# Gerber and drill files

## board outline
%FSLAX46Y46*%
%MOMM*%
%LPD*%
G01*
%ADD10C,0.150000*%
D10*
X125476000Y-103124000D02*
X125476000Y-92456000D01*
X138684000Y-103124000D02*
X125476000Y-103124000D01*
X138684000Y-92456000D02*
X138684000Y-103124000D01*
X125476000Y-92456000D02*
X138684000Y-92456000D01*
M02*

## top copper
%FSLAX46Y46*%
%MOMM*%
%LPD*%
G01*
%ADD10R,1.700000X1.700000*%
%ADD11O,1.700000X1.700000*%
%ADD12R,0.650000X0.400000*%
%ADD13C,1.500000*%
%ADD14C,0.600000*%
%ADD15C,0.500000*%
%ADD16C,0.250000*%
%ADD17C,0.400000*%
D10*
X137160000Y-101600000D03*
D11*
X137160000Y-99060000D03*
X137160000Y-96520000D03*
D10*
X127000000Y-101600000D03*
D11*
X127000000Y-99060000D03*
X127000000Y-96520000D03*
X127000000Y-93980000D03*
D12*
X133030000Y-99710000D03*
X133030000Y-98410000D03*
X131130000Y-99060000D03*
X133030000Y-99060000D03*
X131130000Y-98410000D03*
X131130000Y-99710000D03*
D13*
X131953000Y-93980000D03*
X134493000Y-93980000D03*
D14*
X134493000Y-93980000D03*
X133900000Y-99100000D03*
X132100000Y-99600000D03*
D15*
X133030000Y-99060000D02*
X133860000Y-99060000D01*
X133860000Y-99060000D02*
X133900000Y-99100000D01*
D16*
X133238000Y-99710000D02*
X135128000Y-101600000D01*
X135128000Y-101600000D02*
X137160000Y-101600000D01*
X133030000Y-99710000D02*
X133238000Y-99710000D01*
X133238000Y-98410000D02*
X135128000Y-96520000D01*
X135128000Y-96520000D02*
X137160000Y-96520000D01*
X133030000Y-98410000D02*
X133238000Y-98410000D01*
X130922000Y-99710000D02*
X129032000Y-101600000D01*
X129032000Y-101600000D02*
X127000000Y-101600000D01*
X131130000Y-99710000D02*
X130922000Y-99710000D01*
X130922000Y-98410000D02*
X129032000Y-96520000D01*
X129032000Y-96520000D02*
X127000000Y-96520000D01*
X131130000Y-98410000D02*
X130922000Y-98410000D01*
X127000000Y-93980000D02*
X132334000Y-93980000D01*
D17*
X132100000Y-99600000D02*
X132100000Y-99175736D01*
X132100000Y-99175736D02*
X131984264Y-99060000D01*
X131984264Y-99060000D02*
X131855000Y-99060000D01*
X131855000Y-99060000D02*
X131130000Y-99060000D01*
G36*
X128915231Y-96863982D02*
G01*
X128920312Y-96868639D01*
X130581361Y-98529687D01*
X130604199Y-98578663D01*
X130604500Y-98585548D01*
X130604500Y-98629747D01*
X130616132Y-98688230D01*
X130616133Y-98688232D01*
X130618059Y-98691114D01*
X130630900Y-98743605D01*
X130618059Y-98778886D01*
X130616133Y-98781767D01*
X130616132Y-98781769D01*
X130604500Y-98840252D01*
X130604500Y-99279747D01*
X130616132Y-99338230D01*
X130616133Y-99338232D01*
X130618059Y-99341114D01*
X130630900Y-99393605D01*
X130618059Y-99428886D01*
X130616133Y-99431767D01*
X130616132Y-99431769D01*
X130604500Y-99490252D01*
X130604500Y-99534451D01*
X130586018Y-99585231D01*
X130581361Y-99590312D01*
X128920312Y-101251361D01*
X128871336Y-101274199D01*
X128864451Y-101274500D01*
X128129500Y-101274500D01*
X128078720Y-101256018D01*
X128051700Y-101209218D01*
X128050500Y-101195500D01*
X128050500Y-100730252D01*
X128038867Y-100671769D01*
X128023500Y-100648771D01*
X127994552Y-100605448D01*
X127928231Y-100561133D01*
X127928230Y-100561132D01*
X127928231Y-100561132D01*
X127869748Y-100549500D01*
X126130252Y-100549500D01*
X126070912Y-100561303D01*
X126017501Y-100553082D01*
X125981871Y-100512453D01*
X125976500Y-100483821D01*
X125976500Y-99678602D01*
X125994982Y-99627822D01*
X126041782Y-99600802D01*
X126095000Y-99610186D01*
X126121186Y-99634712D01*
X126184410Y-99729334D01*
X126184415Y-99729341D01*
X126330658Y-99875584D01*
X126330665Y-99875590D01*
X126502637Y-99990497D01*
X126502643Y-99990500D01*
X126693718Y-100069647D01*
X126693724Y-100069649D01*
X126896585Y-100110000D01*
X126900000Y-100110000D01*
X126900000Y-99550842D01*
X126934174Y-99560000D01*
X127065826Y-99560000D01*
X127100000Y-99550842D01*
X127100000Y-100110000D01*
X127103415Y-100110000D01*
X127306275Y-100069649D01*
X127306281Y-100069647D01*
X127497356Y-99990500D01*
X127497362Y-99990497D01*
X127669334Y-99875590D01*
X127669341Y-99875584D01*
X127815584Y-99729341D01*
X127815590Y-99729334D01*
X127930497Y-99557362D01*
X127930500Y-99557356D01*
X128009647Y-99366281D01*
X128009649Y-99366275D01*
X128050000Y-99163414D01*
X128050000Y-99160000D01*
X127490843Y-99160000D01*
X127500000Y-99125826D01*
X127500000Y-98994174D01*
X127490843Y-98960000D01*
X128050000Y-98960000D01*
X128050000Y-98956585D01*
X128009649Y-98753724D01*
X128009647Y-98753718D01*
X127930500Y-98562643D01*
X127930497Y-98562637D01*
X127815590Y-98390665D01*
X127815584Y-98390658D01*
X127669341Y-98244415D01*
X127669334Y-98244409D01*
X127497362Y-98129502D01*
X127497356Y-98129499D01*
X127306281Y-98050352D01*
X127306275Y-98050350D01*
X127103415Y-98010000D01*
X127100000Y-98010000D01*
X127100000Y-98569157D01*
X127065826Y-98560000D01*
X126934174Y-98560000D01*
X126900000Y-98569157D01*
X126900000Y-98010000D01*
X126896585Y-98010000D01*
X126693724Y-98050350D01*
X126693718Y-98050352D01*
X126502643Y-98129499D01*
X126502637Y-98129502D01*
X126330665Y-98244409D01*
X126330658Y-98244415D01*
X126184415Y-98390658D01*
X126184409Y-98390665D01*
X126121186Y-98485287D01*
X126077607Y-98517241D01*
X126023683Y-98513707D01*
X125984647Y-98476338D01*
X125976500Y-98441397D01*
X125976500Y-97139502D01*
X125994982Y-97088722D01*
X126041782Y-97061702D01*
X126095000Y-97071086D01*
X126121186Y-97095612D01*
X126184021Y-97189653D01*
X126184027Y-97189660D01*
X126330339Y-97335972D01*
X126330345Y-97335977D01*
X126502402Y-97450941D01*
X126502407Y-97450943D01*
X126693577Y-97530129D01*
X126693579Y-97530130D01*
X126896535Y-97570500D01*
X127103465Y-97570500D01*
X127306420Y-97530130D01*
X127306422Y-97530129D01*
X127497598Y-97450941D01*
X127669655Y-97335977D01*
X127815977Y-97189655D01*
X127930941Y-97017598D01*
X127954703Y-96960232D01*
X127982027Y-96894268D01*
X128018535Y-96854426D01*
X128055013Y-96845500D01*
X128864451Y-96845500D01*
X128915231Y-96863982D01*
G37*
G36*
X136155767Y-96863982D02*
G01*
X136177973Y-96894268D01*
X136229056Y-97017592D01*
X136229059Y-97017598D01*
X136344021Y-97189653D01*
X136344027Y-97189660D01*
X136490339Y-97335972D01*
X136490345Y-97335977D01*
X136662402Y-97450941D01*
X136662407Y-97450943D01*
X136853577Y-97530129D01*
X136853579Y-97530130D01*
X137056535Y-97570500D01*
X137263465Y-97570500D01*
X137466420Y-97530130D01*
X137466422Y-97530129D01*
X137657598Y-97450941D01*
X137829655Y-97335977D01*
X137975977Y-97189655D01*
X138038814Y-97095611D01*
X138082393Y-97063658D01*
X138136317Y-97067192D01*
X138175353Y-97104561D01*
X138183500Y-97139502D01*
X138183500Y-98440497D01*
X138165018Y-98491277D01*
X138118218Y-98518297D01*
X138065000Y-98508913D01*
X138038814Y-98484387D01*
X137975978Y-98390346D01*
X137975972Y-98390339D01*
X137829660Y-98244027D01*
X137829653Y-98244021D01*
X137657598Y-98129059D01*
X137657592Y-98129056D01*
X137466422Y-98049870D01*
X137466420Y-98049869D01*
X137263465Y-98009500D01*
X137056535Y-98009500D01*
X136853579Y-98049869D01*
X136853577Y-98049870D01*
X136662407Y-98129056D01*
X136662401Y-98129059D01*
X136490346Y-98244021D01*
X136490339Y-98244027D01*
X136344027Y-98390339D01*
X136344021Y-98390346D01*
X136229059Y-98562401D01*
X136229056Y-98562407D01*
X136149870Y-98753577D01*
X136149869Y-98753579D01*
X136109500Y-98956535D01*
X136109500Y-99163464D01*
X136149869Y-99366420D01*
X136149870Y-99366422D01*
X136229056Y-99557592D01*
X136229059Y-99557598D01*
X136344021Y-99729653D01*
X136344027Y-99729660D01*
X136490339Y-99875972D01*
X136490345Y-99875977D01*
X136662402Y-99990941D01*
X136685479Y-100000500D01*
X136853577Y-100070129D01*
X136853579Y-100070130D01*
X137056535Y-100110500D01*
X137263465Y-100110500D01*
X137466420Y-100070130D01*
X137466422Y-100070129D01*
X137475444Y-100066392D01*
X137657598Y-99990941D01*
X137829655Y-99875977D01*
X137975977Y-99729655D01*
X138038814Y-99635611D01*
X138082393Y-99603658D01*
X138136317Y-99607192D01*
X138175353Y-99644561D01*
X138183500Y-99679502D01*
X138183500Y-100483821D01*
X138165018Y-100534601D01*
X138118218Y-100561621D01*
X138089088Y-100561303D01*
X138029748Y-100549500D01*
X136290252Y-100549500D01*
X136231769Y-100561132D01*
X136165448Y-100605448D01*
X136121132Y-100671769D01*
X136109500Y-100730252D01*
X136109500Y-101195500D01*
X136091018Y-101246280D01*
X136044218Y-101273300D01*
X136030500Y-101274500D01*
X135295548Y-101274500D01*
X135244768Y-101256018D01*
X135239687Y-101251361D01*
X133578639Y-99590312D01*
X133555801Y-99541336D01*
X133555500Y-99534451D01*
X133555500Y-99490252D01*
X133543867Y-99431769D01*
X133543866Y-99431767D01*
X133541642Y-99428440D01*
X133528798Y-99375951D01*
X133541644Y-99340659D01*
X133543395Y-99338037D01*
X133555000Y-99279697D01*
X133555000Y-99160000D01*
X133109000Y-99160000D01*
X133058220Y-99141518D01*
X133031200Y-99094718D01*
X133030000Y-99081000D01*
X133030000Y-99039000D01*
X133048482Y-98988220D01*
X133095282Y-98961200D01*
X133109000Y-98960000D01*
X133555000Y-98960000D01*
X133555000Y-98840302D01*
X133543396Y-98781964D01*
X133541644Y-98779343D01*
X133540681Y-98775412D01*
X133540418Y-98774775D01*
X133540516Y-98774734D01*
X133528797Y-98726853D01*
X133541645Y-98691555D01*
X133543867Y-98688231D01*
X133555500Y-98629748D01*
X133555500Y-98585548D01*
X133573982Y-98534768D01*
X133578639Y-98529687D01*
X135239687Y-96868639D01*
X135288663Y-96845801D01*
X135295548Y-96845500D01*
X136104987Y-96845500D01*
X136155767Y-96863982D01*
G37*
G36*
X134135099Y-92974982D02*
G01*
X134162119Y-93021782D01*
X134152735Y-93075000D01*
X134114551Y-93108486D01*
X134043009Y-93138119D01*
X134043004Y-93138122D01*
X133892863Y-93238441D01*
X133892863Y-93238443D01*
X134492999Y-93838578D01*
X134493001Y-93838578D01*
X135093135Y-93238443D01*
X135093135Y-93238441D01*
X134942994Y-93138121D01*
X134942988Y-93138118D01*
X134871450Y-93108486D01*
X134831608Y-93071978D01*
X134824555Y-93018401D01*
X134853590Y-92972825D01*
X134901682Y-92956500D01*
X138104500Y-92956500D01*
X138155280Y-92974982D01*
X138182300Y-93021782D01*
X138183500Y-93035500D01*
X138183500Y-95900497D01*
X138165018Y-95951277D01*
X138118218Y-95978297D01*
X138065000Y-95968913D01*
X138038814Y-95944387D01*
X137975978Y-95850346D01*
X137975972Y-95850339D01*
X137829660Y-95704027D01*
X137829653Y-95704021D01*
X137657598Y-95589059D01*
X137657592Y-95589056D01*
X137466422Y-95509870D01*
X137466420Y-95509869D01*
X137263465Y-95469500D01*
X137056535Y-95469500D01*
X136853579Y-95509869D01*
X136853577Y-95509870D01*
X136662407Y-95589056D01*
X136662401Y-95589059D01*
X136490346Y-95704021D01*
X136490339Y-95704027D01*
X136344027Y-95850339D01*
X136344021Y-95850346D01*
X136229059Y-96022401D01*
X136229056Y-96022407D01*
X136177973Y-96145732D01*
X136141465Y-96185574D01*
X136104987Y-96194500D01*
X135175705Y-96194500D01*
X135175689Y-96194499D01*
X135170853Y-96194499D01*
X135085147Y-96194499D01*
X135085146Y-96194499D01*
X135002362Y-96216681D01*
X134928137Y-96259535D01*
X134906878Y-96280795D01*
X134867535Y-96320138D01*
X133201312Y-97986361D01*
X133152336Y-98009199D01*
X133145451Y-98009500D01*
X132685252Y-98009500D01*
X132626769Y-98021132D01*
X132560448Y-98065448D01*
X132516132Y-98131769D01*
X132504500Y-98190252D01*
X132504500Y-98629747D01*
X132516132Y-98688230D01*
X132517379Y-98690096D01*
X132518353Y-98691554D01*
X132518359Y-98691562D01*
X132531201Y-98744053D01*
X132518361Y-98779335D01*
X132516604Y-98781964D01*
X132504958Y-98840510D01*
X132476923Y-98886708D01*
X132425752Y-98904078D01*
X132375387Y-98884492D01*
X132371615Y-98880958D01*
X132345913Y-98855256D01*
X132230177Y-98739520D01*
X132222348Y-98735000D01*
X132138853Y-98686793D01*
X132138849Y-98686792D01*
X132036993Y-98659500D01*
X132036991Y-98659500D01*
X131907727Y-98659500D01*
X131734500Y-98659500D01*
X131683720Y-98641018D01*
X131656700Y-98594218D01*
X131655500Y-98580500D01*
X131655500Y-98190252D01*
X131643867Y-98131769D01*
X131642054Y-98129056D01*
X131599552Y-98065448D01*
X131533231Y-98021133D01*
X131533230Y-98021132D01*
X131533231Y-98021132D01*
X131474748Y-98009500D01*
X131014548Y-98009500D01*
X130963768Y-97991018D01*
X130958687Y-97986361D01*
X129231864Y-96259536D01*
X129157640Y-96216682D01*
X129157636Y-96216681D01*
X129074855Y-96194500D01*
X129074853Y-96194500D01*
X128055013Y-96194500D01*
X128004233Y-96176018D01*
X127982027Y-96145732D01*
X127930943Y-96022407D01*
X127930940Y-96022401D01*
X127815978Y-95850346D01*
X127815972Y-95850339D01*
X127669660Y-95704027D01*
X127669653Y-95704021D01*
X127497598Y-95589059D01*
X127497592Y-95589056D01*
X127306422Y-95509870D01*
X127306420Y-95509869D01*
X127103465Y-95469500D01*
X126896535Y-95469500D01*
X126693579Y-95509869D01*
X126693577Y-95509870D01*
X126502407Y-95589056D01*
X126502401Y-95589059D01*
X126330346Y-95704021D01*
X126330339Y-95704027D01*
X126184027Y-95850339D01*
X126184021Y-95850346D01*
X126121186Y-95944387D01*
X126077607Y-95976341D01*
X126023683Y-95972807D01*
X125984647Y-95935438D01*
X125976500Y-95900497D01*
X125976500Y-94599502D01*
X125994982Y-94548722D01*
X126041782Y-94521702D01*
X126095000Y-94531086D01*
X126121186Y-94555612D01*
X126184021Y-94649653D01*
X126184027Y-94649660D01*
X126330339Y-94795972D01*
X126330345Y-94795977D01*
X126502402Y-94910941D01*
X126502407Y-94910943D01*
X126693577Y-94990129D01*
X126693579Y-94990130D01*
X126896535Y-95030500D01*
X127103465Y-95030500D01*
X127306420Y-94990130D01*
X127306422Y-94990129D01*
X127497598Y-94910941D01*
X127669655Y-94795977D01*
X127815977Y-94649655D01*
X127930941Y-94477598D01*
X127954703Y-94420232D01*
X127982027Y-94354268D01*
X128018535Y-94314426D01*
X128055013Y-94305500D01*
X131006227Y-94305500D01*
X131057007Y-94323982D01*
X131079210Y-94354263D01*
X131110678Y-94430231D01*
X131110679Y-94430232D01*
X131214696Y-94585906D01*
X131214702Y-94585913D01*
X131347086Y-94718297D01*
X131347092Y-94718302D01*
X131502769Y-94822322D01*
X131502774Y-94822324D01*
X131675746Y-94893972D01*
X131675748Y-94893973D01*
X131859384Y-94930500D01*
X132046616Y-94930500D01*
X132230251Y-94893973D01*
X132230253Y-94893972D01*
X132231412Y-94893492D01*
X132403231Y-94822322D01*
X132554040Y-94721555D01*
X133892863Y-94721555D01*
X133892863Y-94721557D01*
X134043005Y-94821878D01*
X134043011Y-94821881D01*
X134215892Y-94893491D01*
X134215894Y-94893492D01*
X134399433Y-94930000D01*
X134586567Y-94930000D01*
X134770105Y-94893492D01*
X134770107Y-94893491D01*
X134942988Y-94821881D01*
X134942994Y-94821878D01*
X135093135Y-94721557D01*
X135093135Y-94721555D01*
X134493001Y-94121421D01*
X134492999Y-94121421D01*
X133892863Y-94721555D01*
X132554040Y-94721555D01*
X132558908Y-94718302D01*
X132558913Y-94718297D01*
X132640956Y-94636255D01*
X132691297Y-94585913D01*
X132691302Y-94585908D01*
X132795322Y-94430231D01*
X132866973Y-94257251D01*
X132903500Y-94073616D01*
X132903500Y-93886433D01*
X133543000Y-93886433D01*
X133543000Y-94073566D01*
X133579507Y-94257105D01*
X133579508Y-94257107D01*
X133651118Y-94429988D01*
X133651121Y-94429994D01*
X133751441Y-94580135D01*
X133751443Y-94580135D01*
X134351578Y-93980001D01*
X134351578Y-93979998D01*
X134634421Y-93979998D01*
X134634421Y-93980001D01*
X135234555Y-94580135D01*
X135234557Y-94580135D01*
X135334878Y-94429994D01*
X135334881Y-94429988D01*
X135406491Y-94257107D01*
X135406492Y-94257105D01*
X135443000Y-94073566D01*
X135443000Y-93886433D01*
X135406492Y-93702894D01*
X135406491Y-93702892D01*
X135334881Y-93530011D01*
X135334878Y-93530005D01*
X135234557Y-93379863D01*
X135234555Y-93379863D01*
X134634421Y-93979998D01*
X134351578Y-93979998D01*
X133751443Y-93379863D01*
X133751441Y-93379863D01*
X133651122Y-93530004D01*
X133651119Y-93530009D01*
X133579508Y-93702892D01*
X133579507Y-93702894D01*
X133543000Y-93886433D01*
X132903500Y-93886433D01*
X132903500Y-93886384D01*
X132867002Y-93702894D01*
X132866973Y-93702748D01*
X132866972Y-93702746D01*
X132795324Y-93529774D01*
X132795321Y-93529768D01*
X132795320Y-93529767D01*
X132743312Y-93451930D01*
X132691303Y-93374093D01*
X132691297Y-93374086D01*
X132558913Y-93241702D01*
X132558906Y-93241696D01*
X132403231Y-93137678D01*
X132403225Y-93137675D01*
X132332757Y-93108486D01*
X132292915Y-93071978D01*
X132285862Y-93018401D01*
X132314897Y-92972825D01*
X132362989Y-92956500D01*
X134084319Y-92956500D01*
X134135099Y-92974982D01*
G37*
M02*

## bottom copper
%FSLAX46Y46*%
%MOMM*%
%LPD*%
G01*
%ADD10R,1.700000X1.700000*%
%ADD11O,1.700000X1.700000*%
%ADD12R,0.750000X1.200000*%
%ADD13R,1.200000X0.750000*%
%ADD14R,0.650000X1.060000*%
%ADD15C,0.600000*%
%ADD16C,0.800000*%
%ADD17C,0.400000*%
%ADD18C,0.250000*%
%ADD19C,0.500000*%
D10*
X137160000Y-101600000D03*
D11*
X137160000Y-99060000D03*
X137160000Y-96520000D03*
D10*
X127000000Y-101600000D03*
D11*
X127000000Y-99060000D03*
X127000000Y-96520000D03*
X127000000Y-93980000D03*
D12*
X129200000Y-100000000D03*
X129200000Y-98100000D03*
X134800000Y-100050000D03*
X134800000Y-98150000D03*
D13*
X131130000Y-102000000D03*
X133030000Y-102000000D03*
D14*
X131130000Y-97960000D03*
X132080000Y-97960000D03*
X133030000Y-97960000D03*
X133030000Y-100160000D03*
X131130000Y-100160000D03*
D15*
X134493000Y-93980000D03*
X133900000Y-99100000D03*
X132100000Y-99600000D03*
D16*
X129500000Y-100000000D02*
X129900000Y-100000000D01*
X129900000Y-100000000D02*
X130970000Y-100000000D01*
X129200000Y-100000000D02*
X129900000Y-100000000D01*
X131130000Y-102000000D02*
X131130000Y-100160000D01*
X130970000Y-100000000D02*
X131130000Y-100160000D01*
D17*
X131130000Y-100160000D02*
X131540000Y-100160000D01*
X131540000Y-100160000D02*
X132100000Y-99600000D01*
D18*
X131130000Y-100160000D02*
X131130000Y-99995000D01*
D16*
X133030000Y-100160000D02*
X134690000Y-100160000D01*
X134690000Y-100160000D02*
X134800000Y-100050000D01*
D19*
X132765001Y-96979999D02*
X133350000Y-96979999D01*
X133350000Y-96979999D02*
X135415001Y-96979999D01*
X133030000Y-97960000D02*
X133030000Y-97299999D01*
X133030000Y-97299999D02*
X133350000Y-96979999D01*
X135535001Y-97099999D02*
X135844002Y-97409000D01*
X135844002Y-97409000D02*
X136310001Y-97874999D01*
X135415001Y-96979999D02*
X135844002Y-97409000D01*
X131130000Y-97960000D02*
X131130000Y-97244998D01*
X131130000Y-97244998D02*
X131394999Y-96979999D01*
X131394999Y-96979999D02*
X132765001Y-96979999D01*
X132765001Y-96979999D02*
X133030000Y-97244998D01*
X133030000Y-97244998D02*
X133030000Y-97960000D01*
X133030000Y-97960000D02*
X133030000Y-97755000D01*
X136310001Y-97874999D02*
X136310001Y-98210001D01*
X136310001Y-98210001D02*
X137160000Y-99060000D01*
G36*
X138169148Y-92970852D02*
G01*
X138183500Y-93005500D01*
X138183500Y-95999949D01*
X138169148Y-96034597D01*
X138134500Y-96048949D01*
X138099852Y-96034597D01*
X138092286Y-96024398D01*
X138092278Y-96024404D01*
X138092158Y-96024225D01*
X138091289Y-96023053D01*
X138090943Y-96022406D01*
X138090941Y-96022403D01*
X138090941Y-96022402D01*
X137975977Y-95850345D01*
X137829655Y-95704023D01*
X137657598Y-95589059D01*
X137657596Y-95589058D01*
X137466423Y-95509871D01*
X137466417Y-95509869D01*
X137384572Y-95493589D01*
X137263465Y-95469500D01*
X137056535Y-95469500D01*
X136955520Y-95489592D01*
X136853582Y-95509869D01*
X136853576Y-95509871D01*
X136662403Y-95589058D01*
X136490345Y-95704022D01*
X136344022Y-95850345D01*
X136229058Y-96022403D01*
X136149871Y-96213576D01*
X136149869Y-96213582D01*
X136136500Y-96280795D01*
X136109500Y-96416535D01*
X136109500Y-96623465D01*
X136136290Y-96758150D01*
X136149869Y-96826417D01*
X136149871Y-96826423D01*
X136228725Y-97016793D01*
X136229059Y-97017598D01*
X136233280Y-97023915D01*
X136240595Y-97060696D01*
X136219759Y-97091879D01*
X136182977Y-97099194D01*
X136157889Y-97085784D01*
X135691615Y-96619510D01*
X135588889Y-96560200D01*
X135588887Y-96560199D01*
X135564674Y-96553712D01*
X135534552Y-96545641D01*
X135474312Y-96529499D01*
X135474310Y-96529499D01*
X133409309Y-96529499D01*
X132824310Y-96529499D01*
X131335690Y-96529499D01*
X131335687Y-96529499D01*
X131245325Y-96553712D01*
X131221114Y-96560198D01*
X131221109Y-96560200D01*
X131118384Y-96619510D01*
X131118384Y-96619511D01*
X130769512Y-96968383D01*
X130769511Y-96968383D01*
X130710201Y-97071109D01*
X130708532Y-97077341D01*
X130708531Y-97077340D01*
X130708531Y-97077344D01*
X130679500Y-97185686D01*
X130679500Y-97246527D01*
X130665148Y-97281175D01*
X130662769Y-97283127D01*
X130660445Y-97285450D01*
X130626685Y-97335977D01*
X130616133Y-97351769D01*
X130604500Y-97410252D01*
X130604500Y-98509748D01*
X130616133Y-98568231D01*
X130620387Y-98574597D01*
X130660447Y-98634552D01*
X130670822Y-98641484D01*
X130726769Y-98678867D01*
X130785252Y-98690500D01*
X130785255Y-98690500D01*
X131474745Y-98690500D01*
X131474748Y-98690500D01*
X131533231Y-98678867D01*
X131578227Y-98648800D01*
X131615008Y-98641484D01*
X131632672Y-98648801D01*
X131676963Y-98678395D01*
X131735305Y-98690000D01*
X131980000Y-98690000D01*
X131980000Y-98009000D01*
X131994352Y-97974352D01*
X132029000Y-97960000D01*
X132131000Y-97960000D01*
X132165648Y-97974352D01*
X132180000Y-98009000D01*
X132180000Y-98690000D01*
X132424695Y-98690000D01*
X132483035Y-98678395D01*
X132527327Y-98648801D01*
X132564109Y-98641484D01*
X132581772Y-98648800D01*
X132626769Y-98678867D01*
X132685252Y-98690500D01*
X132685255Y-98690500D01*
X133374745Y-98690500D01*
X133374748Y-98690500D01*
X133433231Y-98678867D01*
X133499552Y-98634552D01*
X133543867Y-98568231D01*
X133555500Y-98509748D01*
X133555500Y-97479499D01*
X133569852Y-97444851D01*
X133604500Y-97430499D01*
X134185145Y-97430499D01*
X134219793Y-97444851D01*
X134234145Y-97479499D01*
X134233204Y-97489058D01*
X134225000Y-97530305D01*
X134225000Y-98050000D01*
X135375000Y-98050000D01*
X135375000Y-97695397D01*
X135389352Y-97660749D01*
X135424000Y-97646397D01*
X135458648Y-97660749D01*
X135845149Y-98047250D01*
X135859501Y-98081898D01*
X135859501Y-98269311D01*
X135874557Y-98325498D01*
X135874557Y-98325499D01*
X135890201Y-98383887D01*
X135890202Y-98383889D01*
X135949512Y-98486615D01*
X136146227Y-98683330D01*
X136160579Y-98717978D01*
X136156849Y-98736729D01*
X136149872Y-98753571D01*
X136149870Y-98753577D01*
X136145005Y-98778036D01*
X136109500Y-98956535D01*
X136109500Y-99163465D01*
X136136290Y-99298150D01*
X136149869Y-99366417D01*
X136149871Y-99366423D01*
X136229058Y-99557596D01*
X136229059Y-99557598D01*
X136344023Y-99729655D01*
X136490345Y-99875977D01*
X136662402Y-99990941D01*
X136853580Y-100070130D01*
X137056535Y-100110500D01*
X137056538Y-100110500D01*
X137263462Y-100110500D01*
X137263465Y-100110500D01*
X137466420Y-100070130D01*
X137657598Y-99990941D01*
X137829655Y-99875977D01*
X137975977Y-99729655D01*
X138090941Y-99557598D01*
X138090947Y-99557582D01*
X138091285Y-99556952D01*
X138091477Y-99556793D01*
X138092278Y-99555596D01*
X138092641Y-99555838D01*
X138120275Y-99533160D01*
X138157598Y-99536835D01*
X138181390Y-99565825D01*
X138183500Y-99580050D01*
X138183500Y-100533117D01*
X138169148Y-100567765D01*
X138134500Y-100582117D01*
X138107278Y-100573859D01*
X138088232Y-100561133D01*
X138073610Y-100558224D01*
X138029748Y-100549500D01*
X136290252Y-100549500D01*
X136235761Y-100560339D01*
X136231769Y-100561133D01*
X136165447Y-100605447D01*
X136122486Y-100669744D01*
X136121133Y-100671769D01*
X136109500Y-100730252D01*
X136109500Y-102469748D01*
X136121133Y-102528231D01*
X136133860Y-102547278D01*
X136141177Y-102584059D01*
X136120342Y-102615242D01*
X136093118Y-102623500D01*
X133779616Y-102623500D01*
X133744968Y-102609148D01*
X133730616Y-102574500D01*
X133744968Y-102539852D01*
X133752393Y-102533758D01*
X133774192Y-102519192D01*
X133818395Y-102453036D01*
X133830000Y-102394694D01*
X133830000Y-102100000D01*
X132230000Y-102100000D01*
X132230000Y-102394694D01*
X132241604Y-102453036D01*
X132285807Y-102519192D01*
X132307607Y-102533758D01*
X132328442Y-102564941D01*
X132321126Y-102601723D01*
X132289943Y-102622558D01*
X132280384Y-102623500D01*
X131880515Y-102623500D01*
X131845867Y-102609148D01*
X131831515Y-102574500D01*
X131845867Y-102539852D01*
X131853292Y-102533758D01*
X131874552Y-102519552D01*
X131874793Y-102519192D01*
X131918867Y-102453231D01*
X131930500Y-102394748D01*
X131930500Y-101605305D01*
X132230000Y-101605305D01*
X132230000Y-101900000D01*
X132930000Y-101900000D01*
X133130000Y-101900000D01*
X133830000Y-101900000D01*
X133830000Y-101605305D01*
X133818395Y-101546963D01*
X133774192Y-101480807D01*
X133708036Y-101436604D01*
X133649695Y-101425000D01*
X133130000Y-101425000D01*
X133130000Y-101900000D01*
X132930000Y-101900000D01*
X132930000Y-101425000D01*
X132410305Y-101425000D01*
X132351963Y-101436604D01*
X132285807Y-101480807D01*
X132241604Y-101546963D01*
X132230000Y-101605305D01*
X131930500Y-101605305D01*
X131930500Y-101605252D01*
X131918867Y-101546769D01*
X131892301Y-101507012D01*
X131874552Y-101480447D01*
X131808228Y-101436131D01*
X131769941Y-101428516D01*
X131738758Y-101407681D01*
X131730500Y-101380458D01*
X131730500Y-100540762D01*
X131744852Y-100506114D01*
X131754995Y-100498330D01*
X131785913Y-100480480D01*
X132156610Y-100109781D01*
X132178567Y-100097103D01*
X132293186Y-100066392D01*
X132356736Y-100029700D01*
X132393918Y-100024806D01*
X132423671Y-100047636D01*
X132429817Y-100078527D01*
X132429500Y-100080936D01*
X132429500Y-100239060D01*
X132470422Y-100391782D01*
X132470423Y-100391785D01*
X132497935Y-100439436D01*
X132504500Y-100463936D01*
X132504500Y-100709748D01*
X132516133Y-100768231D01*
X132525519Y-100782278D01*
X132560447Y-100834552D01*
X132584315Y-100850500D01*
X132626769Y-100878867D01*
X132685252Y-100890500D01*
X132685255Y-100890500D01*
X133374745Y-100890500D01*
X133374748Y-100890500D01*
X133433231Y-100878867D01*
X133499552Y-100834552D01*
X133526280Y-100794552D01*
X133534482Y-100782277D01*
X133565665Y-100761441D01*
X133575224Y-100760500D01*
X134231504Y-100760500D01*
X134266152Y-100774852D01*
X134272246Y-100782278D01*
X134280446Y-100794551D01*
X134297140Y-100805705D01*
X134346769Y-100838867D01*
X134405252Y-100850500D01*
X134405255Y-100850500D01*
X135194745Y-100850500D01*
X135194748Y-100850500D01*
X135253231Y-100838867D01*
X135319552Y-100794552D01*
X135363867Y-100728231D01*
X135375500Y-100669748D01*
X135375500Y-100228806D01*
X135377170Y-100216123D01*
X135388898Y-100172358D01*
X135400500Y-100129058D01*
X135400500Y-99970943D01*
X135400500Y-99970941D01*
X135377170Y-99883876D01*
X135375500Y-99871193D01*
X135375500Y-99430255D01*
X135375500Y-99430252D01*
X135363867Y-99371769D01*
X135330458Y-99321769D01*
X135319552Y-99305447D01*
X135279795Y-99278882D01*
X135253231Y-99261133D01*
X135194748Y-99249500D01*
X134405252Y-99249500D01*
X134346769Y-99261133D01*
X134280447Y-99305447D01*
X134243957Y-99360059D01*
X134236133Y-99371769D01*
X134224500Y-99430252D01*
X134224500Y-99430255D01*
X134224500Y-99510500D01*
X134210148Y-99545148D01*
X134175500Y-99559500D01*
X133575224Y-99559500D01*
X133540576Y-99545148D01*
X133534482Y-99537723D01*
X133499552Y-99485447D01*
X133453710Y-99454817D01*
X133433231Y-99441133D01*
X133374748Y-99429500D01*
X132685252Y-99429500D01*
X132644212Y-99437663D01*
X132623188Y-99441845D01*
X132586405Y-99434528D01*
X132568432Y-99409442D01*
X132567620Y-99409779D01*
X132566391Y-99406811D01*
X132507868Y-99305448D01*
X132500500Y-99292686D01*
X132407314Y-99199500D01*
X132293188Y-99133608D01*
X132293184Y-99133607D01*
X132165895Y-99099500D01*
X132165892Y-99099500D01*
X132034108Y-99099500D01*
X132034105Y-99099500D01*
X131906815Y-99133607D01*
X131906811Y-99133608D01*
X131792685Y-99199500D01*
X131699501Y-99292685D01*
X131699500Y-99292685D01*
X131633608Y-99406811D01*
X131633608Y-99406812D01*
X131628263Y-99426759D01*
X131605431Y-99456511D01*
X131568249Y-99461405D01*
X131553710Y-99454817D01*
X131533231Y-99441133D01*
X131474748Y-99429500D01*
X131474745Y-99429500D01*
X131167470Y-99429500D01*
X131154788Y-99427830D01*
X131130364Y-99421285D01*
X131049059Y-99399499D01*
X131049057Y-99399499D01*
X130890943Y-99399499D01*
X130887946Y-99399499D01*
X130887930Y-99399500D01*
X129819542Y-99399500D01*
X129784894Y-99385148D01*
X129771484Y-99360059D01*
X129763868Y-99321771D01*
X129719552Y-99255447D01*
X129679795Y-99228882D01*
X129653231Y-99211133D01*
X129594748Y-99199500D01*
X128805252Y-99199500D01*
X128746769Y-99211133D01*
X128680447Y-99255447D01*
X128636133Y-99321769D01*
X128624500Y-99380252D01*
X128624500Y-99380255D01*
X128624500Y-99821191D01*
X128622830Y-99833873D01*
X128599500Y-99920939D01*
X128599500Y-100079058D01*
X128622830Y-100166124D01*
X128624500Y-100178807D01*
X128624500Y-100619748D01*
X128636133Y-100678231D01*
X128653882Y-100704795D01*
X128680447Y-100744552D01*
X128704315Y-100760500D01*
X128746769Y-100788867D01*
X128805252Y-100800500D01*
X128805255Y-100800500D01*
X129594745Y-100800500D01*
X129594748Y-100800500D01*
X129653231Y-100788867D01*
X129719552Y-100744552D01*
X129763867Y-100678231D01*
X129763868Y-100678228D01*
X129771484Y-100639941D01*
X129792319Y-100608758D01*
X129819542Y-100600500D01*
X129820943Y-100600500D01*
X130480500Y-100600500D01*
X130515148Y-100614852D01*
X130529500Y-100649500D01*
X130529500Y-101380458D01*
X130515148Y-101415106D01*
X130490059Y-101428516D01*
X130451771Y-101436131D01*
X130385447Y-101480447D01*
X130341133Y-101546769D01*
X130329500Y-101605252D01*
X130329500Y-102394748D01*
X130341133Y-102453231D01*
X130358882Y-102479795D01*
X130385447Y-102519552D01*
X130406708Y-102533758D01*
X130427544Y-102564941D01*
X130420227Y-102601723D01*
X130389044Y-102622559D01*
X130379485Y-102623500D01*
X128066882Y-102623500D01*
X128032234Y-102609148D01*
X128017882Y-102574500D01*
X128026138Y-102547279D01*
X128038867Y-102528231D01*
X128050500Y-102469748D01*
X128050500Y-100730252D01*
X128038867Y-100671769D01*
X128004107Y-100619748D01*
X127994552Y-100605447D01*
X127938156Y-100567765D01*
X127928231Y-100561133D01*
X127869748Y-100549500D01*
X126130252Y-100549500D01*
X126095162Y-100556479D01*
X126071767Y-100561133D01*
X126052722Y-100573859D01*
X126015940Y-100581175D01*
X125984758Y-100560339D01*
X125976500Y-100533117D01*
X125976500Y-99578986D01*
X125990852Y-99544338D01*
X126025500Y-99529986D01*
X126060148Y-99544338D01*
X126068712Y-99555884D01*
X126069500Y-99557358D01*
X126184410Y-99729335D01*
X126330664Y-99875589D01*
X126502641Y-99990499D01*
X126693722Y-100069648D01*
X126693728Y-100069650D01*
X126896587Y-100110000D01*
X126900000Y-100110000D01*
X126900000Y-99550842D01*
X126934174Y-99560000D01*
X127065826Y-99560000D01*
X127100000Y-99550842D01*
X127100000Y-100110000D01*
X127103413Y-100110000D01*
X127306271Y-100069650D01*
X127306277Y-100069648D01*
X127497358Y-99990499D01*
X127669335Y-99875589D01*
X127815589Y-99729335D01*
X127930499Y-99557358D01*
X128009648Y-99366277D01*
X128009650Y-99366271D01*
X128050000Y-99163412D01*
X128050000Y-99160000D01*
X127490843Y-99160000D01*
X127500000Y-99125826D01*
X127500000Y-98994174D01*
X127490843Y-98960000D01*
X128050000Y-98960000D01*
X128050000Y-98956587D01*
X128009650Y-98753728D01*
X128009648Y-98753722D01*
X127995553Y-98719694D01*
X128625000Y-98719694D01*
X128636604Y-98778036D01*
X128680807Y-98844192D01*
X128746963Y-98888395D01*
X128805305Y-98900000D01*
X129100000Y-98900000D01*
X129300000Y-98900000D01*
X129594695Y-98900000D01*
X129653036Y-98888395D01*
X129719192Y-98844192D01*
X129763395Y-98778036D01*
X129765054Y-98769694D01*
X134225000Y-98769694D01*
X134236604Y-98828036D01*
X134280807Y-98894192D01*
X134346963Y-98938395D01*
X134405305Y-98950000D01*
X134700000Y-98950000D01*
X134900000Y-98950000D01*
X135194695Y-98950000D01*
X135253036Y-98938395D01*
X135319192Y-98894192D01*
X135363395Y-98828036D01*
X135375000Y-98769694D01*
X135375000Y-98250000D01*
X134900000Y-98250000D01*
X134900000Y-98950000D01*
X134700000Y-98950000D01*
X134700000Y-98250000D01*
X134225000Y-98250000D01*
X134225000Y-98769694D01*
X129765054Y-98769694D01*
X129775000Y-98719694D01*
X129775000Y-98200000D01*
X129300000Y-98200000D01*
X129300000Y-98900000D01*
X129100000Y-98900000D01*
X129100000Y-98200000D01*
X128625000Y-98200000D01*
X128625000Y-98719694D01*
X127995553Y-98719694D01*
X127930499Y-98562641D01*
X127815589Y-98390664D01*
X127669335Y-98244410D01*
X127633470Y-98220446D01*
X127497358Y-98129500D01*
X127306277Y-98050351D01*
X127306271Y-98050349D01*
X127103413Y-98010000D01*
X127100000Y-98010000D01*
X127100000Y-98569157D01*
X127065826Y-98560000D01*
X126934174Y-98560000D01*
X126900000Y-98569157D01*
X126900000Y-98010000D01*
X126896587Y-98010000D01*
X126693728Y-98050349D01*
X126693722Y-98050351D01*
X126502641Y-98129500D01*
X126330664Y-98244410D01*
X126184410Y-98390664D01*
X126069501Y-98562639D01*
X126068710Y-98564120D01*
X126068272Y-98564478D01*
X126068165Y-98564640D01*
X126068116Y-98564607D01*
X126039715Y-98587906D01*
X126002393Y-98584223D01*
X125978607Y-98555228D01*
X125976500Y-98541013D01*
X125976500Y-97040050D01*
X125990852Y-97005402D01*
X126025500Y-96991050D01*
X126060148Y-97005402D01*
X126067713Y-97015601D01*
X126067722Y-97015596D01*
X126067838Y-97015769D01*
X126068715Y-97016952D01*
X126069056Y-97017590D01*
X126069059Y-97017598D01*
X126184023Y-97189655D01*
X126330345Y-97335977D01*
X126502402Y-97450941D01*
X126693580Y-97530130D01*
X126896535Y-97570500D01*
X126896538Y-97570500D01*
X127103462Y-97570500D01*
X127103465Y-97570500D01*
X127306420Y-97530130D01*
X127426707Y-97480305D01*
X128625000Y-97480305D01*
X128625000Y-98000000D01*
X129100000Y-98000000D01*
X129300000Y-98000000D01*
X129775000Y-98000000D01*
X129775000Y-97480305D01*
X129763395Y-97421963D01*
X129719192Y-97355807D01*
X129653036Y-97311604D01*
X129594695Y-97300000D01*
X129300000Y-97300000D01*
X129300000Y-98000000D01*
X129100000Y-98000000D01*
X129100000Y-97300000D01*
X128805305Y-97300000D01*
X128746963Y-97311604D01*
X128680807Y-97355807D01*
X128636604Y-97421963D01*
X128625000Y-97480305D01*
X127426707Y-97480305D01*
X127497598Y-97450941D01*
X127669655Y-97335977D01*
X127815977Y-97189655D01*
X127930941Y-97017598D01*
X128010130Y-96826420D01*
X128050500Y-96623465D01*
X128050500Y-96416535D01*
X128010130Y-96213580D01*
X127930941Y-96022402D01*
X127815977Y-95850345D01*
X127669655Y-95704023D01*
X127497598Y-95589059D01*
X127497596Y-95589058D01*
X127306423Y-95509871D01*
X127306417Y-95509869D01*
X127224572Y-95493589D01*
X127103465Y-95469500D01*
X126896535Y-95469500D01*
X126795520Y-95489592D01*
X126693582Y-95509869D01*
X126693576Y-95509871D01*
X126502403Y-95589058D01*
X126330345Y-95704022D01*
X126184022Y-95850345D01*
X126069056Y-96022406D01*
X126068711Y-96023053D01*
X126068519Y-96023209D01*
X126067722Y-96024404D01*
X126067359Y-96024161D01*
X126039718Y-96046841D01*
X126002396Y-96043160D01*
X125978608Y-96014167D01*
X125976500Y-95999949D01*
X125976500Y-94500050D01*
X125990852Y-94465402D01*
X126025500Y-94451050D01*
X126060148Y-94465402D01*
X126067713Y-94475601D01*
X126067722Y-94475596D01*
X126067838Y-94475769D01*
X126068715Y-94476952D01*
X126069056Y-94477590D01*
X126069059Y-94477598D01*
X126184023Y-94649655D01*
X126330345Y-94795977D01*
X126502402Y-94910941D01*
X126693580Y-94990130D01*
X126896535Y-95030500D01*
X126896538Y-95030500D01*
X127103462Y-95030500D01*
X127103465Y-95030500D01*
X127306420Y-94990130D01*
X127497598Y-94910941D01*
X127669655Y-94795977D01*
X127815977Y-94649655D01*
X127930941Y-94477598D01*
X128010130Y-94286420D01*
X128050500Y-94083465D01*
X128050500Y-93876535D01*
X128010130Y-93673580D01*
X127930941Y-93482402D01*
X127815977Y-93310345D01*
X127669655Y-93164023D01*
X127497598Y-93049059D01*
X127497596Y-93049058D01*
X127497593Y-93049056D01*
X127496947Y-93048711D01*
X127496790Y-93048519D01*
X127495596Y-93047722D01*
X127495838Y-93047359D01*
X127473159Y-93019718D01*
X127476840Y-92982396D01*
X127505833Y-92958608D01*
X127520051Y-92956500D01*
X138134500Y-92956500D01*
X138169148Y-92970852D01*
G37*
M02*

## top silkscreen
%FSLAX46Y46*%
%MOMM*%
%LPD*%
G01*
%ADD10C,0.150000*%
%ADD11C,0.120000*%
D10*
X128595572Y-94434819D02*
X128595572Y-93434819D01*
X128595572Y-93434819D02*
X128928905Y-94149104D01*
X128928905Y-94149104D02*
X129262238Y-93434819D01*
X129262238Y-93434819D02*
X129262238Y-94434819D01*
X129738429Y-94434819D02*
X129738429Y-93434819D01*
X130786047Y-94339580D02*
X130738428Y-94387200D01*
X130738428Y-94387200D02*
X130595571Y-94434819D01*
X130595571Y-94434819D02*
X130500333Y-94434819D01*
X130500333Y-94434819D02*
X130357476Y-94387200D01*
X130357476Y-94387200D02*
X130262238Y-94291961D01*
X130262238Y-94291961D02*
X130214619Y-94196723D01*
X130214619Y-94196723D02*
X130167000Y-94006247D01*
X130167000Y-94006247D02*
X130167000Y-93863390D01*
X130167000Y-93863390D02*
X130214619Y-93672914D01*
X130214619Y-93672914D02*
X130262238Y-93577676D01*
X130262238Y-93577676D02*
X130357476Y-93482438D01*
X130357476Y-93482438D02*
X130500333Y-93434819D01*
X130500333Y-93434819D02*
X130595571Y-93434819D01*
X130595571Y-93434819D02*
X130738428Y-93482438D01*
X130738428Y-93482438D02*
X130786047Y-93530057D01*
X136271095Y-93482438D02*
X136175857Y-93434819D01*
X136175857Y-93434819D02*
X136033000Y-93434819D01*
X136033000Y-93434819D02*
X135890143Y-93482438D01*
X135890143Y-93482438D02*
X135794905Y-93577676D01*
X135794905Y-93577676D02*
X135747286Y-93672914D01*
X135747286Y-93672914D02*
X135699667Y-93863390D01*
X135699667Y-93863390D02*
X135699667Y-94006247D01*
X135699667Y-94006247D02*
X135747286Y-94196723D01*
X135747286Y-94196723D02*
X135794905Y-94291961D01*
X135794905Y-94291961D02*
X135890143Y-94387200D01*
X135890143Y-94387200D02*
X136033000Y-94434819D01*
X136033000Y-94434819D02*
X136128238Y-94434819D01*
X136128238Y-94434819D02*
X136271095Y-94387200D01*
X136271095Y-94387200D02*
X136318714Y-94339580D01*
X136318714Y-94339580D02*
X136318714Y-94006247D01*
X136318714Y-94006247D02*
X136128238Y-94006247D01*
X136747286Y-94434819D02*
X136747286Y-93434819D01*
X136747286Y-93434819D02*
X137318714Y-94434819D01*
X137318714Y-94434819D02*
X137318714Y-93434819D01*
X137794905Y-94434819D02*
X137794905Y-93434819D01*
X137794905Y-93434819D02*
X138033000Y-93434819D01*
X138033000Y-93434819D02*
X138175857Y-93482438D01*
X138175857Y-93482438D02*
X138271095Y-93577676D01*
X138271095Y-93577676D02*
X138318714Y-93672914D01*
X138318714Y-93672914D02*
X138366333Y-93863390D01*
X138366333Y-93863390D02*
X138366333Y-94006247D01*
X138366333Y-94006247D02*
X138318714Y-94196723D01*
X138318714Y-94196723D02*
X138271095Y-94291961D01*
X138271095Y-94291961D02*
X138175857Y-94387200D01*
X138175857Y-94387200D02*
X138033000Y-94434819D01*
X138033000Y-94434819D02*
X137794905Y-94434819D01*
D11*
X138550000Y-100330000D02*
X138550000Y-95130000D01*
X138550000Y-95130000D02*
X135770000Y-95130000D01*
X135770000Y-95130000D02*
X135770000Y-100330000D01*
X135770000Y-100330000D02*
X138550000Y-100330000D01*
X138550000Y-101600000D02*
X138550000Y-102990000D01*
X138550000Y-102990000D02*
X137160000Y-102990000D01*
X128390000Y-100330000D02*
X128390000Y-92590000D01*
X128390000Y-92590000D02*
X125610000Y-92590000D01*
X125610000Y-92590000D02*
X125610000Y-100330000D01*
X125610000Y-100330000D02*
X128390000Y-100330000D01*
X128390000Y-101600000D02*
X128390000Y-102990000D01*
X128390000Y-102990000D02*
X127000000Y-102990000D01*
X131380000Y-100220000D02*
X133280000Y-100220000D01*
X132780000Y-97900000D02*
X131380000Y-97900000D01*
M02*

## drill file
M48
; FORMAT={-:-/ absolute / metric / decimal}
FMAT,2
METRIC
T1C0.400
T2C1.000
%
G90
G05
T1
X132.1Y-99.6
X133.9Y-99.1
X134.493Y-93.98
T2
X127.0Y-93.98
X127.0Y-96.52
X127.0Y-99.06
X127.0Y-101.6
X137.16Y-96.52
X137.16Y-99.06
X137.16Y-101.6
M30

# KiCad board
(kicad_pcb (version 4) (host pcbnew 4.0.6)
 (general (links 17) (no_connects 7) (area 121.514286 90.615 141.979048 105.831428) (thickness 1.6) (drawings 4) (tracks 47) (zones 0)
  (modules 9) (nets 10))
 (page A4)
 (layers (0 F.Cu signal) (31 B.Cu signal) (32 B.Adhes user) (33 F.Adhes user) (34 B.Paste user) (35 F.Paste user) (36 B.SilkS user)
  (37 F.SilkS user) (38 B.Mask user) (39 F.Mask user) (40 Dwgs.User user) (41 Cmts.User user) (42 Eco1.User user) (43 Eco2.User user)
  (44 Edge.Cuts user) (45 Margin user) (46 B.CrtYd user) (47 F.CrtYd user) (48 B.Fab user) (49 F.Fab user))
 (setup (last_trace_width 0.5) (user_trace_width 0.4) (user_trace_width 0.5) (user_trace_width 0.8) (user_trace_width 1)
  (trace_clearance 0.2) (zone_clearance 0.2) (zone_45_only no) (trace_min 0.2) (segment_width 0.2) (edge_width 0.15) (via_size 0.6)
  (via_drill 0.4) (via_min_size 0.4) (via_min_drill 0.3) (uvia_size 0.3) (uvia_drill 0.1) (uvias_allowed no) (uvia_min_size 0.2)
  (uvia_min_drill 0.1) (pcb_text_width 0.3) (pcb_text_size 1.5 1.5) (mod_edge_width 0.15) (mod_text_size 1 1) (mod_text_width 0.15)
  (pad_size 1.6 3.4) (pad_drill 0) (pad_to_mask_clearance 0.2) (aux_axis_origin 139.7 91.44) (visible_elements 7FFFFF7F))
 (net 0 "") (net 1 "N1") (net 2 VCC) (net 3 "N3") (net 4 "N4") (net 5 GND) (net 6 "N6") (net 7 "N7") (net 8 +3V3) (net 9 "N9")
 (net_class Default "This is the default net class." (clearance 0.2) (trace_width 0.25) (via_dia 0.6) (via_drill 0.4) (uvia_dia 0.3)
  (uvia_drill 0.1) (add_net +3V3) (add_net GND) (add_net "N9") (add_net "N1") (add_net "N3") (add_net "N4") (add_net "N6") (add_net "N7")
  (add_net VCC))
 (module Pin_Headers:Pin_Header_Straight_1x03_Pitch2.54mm (layer F.Cu) (at 137.16 101.6 180)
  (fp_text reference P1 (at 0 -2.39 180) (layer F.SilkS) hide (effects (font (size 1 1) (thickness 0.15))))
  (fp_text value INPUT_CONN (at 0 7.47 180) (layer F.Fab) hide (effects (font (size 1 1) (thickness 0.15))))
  (fp_line (start -1.39 1.27) (end -1.39 6.47) (layer F.SilkS) (width 0.12))
  (fp_line (start -1.39 6.47) (end 1.39 6.47) (layer F.SilkS) (width 0.12))
  (fp_line (start 1.39 6.47) (end 1.39 1.27) (layer F.SilkS) (width 0.12))
  (fp_line (start 1.39 1.27) (end -1.39 1.27) (layer F.SilkS) (width 0.12))
  (fp_line (start -1.39 0) (end -1.39 -1.39) (layer F.SilkS) (width 0.12))
  (fp_line (start -1.39 -1.39) (end 0 -1.39) (layer F.SilkS) (width 0.12))
  (pad 1 thru_hole rect (at 0 0 180) (size 1.7 1.7) (drill 1) (layers *.Cu *.Mask) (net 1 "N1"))
  (pad 2 thru_hole oval (at 0 2.54 180) (size 1.7 1.7) (drill 1) (layers *.Cu *.Mask) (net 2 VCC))
  (pad 3 thru_hole oval (at 0 5.08 180) (size 1.7 1.7) (drill 1) (layers *.Cu *.Mask) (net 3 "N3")))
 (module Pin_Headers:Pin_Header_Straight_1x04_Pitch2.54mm (layer F.Cu) (at 127 101.6 180)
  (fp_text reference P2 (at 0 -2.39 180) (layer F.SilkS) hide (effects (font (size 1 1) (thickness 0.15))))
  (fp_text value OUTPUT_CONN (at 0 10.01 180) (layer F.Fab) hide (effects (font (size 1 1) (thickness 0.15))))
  (fp_line (start -1.39 1.27) (end -1.39 9.01) (layer F.SilkS) (width 0.12))
  (fp_line (start -1.39 9.01) (end 1.39 9.01) (layer F.SilkS) (width 0.12))
  (fp_line (start 1.39 9.01) (end 1.39 1.27) (layer F.SilkS) (width 0.12))
  (fp_line (start 1.39 1.27) (end -1.39 1.27) (layer F.SilkS) (width 0.12))
  (fp_line (start -1.39 0) (end -1.39 -1.39) (layer F.SilkS) (width 0.12))
  (fp_line (start -1.39 -1.39) (end 0 -1.39) (layer F.SilkS) (width 0.12))
  (pad 1 thru_hole rect (at 0 0 180) (size 1.7 1.7) (drill 1) (layers *.Cu *.Mask) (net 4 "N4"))
  (pad 2 thru_hole oval (at 0 2.54 180) (size 1.7 1.7) (drill 1) (layers *.Cu *.Mask) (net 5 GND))
  (pad 3 thru_hole oval (at 0 5.08 180) (size 1.7 1.7) (drill 1) (layers *.Cu *.Mask) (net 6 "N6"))
  (pad 4 thru_hole oval (at 0 7.62 180) (size 1.7 1.7) (drill 1) (layers *.Cu *.Mask) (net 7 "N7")))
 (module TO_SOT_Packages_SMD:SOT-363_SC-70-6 (layer F.Cu) (at 132.08 99.06 180)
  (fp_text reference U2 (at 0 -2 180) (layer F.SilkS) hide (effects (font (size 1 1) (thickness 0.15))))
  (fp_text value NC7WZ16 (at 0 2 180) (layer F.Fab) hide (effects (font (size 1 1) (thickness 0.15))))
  (fp_line (start 0.7 -1.16) (end -1.2 -1.16) (layer F.SilkS) (width 0.12))
  (fp_line (start -0.7 1.16) (end 0.7 1.16) (layer F.SilkS) (width 0.12))
  (pad 1 smd rect (at -0.95 -0.65 180) (size 0.65 0.4) (layers F.Cu F.Paste F.Mask) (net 1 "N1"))
  (pad 3 smd rect (at -0.95 0.65 180) (size 0.65 0.4) (layers F.Cu F.Paste F.Mask) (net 3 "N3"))
  (pad 5 smd rect (at 0.95 0 180) (size 0.65 0.4) (layers F.Cu F.Paste F.Mask) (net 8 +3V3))
  (pad 2 smd rect (at -0.95 0 180) (size 0.65 0.4) (layers F.Cu F.Paste F.Mask) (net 5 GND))
  (pad 4 smd rect (at 0.95 0.65 180) (size 0.65 0.4) (layers F.Cu F.Paste F.Mask) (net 6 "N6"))
  (pad 6 smd rect (at 0.95 -0.65 180) (size 0.65 0.4) (layers F.Cu F.Paste F.Mask) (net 4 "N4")))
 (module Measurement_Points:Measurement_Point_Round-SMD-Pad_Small (layer F.Cu) (at 131.953 93.98)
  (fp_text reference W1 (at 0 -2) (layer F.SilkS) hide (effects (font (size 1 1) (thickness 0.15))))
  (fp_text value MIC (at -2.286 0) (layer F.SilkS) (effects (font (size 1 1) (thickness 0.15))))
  (pad 1 smd circle (at 0 0) (size 1.5 1.5) (layers F.Cu F.Mask) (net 7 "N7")))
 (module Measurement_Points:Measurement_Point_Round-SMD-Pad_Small (layer F.Cu) (at 134.493 93.98)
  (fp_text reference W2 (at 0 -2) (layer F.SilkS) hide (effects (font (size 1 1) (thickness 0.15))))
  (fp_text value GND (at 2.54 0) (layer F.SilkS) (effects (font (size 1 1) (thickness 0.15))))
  (pad 1 smd circle (at 0 0) (size 1.5 1.5) (layers F.Cu F.Mask) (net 5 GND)))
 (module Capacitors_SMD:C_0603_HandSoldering (layer B.Cu) (at 129.2 99.05 90)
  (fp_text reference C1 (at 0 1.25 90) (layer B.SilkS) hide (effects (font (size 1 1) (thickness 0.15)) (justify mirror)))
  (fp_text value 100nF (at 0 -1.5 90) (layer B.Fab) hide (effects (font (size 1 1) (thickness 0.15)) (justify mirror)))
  (pad 1 smd rect (at -0.95 0 90) (size 1.2 0.75) (layers B.Cu B.Paste B.Mask) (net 8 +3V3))
  (pad 2 smd rect (at 0.95 0 90) (size 1.2 0.75) (layers B.Cu B.Paste B.Mask) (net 5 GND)))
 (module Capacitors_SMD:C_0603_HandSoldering (layer B.Cu) (at 134.8 99.1 90)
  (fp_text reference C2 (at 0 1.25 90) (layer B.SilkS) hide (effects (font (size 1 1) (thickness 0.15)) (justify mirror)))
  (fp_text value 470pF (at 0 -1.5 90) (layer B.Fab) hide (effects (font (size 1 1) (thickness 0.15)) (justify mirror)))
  (pad 1 smd rect (at -0.95 0 90) (size 1.2 0.75) (layers B.Cu B.Paste B.Mask) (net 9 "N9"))
  (pad 2 smd rect (at 0.95 0 90) (size 1.2 0.75) (layers B.Cu B.Paste B.Mask) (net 5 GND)))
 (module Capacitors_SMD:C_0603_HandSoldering (layer B.Cu) (at 132.08 102)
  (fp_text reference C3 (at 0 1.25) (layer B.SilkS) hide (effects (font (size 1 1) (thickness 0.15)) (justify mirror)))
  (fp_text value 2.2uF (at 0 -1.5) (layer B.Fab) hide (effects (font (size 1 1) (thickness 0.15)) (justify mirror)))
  (pad 1 smd rect (at -0.95 0) (size 1.2 0.75) (layers B.Cu B.Paste B.Mask) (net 8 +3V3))
  (pad 2 smd rect (at 0.95 0) (size 1.2 0.75) (layers B.Cu B.Paste B.Mask) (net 5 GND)))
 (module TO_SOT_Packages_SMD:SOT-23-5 (layer B.Cu) (at 132.08 99.06 270)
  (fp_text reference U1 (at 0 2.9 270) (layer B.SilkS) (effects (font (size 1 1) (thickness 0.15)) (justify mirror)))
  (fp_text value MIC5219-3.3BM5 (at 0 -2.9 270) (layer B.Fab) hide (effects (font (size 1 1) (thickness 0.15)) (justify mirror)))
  (pad 1 smd rect (at -1.1 0.95 270) (size 1.06 0.65) (layers B.Cu B.Paste B.Mask) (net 2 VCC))
  (pad 2 smd rect (at -1.1 0 270) (size 1.06 0.65) (layers B.Cu B.Paste B.Mask) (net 5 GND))
  (pad 3 smd rect (at -1.1 -0.95 270) (size 1.06 0.65) (layers B.Cu B.Paste B.Mask) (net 2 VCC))
  (pad 4 smd rect (at 1.1 -0.95 270) (size 1.06 0.65) (layers B.Cu B.Paste B.Mask) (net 9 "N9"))
  (pad 5 smd rect (at 1.1 0.95 270) (size 1.06 0.65) (layers B.Cu B.Paste B.Mask) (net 8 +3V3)))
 (gr_line (start 125.476 103.124) (end 125.476 92.456) (layer Edge.Cuts) (width 0.15))
 (gr_line (start 138.684 103.124) (end 125.476 103.124) (layer Edge.Cuts) (width 0.15))
 (gr_line (start 138.684 92.456) (end 138.684 103.124) (layer Edge.Cuts) (width 0.15))
 (gr_line (start 125.476 92.456) (end 138.684 92.456) (layer Edge.Cuts) (width 0.15))
 (via (at 134.493 93.98) (size 0.6) (drill 0.4) (layers F.Cu B.Cu) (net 5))
 (segment (start 133.03 99.06) (end 133.86 99.06) (width 0.5) (layer F.Cu) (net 5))
 (segment (start 133.86 99.06) (end 133.9 99.1) (width 0.5) (layer F.Cu) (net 5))
 (via (at 133.9 99.1) (size 0.6) (drill 0.4) (layers F.Cu B.Cu) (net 5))
 (segment (start 133.238 99.71) (end 135.128 101.6) (width 0.25) (layer F.Cu) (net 1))
 (segment (start 135.128 101.6) (end 137.16 101.6) (width 0.25) (layer F.Cu) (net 1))
 (segment (start 133.03 99.71) (end 133.238 99.71) (width 0.25) (layer F.Cu) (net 1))
 (segment (start 133.238 98.41) (end 135.128 96.52) (width 0.25) (layer F.Cu) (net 3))
 (segment (start 135.128 96.52) (end 137.16 96.52) (width 0.25) (layer F.Cu) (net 3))
 (segment (start 133.03 98.41) (end 133.238 98.41) (width 0.25) (layer F.Cu) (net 3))
 (segment (start 130.922 99.71) (end 129.032 101.6) (width 0.25) (layer F.Cu) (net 4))
 (segment (start 129.032 101.6) (end 127 101.6) (width 0.25) (layer F.Cu) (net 4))
 (segment (start 131.13 99.71) (end 130.922 99.71) (width 0.25) (layer F.Cu) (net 4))
 (segment (start 130.922 98.41) (end 129.032 96.52) (width 0.25) (layer F.Cu) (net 6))
 (segment (start 129.032 96.52) (end 127 96.52) (width 0.25) (layer F.Cu) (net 6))
 (segment (start 131.13 98.41) (end 130.922 98.41) (width 0.25) (layer F.Cu) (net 6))
 (segment (start 127 93.98) (end 132.334 93.98) (width 0.25) (layer F.Cu) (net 7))
 (segment (start 129.5 100) (end 129.9 100) (width 0.8) (layer B.Cu) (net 8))
 (segment (start 129.9 100) (end 130.97 100) (width 0.8) (layer B.Cu) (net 8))
 (segment (start 129.2 100) (end 129.9 100) (width 0.8) (layer B.Cu) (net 8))
 (segment (start 131.13 102) (end 131.13 100.16) (width 0.8) (layer B.Cu) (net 8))
 (segment (start 130.97 100) (end 131.13 100.16) (width 0.8) (layer B.Cu) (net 8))
 (segment (start 132.1 99.6) (end 132.1 99.175736) (width 0.4) (layer F.Cu) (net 8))
 (segment (start 132.1 99.175736) (end 131.984264 99.06) (width 0.4) (layer F.Cu) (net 8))
 (segment (start 131.984264 99.06) (end 131.855 99.06) (width 0.4) (layer F.Cu) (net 8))
 (segment (start 131.855 99.06) (end 131.13 99.06) (width 0.4) (layer F.Cu) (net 8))
 (segment (start 131.13 100.16) (end 131.54 100.16) (width 0.4) (layer B.Cu) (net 8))
 (segment (start 131.54 100.16) (end 132.1 99.6) (width 0.4) (layer B.Cu) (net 8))
 (via (at 132.1 99.6) (size 0.6) (drill 0.4) (layers F.Cu B.Cu) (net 8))
 (segment (start 131.13 100.16) (end 131.13 99.995) (width 0.25) (layer B.Cu) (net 8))
 (segment (start 133.03 100.16) (end 134.69 100.16) (width 0.8) (layer B.Cu) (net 9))
 (segment (start 134.69 100.16) (end 134.8 100.05) (width 0.8) (layer B.Cu) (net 9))
 (segment (start 132.765001 96.979999) (end 133.35 96.979999) (width 0.5) (layer B.Cu) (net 2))
 (segment (start 133.35 96.979999) (end 135.415001 96.979999) (width 0.5) (layer B.Cu) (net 2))
 (segment (start 133.03 97.96) (end 133.03 97.299999) (width 0.5) (layer B.Cu) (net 2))
 (segment (start 133.03 97.299999) (end 133.35 96.979999) (width 0.5) (layer B.Cu) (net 2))
 (segment (start 135.535001 97.099999) (end 135.844002 97.409) (width 0.5) (layer B.Cu) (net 2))
 (segment (start 135.844002 97.409) (end 136.310001 97.874999) (width 0.5) (layer B.Cu) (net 2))
 (segment (start 135.415001 96.979999) (end 135.844002 97.409) (width 0.5) (layer B.Cu) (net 2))
 (segment (start 131.13 97.96) (end 131.13 97.244998) (width 0.5) (layer B.Cu) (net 2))
 (segment (start 131.13 97.244998) (end 131.394999 96.979999) (width 0.5) (layer B.Cu) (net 2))
 (segment (start 131.394999 96.979999) (end 132.765001 96.979999) (width 0.5) (layer B.Cu) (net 2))
 (segment (start 132.765001 96.979999) (end 133.03 97.244998) (width 0.5) (layer B.Cu) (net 2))
 (segment (start 133.03 97.244998) (end 133.03 97.96) (width 0.5) (layer B.Cu) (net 2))
 (segment (start 133.03 97.96) (end 133.03 97.755) (width 0.5) (layer B.Cu) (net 2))
 (segment (start 136.310001 97.874999) (end 136.310001 98.210001) (width 0.5) (layer B.Cu) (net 2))
 (segment (start 136.310001 98.210001) (end 137.16 99.06) (width 0.5) (layer B.Cu) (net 2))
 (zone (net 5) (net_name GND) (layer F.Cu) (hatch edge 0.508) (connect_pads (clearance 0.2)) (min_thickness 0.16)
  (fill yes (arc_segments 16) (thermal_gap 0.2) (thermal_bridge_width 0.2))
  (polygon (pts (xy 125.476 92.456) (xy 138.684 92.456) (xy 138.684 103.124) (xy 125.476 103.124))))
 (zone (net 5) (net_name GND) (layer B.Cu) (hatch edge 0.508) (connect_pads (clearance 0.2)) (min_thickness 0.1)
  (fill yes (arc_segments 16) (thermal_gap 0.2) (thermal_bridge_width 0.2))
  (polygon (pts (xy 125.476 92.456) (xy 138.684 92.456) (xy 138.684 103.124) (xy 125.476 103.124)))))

